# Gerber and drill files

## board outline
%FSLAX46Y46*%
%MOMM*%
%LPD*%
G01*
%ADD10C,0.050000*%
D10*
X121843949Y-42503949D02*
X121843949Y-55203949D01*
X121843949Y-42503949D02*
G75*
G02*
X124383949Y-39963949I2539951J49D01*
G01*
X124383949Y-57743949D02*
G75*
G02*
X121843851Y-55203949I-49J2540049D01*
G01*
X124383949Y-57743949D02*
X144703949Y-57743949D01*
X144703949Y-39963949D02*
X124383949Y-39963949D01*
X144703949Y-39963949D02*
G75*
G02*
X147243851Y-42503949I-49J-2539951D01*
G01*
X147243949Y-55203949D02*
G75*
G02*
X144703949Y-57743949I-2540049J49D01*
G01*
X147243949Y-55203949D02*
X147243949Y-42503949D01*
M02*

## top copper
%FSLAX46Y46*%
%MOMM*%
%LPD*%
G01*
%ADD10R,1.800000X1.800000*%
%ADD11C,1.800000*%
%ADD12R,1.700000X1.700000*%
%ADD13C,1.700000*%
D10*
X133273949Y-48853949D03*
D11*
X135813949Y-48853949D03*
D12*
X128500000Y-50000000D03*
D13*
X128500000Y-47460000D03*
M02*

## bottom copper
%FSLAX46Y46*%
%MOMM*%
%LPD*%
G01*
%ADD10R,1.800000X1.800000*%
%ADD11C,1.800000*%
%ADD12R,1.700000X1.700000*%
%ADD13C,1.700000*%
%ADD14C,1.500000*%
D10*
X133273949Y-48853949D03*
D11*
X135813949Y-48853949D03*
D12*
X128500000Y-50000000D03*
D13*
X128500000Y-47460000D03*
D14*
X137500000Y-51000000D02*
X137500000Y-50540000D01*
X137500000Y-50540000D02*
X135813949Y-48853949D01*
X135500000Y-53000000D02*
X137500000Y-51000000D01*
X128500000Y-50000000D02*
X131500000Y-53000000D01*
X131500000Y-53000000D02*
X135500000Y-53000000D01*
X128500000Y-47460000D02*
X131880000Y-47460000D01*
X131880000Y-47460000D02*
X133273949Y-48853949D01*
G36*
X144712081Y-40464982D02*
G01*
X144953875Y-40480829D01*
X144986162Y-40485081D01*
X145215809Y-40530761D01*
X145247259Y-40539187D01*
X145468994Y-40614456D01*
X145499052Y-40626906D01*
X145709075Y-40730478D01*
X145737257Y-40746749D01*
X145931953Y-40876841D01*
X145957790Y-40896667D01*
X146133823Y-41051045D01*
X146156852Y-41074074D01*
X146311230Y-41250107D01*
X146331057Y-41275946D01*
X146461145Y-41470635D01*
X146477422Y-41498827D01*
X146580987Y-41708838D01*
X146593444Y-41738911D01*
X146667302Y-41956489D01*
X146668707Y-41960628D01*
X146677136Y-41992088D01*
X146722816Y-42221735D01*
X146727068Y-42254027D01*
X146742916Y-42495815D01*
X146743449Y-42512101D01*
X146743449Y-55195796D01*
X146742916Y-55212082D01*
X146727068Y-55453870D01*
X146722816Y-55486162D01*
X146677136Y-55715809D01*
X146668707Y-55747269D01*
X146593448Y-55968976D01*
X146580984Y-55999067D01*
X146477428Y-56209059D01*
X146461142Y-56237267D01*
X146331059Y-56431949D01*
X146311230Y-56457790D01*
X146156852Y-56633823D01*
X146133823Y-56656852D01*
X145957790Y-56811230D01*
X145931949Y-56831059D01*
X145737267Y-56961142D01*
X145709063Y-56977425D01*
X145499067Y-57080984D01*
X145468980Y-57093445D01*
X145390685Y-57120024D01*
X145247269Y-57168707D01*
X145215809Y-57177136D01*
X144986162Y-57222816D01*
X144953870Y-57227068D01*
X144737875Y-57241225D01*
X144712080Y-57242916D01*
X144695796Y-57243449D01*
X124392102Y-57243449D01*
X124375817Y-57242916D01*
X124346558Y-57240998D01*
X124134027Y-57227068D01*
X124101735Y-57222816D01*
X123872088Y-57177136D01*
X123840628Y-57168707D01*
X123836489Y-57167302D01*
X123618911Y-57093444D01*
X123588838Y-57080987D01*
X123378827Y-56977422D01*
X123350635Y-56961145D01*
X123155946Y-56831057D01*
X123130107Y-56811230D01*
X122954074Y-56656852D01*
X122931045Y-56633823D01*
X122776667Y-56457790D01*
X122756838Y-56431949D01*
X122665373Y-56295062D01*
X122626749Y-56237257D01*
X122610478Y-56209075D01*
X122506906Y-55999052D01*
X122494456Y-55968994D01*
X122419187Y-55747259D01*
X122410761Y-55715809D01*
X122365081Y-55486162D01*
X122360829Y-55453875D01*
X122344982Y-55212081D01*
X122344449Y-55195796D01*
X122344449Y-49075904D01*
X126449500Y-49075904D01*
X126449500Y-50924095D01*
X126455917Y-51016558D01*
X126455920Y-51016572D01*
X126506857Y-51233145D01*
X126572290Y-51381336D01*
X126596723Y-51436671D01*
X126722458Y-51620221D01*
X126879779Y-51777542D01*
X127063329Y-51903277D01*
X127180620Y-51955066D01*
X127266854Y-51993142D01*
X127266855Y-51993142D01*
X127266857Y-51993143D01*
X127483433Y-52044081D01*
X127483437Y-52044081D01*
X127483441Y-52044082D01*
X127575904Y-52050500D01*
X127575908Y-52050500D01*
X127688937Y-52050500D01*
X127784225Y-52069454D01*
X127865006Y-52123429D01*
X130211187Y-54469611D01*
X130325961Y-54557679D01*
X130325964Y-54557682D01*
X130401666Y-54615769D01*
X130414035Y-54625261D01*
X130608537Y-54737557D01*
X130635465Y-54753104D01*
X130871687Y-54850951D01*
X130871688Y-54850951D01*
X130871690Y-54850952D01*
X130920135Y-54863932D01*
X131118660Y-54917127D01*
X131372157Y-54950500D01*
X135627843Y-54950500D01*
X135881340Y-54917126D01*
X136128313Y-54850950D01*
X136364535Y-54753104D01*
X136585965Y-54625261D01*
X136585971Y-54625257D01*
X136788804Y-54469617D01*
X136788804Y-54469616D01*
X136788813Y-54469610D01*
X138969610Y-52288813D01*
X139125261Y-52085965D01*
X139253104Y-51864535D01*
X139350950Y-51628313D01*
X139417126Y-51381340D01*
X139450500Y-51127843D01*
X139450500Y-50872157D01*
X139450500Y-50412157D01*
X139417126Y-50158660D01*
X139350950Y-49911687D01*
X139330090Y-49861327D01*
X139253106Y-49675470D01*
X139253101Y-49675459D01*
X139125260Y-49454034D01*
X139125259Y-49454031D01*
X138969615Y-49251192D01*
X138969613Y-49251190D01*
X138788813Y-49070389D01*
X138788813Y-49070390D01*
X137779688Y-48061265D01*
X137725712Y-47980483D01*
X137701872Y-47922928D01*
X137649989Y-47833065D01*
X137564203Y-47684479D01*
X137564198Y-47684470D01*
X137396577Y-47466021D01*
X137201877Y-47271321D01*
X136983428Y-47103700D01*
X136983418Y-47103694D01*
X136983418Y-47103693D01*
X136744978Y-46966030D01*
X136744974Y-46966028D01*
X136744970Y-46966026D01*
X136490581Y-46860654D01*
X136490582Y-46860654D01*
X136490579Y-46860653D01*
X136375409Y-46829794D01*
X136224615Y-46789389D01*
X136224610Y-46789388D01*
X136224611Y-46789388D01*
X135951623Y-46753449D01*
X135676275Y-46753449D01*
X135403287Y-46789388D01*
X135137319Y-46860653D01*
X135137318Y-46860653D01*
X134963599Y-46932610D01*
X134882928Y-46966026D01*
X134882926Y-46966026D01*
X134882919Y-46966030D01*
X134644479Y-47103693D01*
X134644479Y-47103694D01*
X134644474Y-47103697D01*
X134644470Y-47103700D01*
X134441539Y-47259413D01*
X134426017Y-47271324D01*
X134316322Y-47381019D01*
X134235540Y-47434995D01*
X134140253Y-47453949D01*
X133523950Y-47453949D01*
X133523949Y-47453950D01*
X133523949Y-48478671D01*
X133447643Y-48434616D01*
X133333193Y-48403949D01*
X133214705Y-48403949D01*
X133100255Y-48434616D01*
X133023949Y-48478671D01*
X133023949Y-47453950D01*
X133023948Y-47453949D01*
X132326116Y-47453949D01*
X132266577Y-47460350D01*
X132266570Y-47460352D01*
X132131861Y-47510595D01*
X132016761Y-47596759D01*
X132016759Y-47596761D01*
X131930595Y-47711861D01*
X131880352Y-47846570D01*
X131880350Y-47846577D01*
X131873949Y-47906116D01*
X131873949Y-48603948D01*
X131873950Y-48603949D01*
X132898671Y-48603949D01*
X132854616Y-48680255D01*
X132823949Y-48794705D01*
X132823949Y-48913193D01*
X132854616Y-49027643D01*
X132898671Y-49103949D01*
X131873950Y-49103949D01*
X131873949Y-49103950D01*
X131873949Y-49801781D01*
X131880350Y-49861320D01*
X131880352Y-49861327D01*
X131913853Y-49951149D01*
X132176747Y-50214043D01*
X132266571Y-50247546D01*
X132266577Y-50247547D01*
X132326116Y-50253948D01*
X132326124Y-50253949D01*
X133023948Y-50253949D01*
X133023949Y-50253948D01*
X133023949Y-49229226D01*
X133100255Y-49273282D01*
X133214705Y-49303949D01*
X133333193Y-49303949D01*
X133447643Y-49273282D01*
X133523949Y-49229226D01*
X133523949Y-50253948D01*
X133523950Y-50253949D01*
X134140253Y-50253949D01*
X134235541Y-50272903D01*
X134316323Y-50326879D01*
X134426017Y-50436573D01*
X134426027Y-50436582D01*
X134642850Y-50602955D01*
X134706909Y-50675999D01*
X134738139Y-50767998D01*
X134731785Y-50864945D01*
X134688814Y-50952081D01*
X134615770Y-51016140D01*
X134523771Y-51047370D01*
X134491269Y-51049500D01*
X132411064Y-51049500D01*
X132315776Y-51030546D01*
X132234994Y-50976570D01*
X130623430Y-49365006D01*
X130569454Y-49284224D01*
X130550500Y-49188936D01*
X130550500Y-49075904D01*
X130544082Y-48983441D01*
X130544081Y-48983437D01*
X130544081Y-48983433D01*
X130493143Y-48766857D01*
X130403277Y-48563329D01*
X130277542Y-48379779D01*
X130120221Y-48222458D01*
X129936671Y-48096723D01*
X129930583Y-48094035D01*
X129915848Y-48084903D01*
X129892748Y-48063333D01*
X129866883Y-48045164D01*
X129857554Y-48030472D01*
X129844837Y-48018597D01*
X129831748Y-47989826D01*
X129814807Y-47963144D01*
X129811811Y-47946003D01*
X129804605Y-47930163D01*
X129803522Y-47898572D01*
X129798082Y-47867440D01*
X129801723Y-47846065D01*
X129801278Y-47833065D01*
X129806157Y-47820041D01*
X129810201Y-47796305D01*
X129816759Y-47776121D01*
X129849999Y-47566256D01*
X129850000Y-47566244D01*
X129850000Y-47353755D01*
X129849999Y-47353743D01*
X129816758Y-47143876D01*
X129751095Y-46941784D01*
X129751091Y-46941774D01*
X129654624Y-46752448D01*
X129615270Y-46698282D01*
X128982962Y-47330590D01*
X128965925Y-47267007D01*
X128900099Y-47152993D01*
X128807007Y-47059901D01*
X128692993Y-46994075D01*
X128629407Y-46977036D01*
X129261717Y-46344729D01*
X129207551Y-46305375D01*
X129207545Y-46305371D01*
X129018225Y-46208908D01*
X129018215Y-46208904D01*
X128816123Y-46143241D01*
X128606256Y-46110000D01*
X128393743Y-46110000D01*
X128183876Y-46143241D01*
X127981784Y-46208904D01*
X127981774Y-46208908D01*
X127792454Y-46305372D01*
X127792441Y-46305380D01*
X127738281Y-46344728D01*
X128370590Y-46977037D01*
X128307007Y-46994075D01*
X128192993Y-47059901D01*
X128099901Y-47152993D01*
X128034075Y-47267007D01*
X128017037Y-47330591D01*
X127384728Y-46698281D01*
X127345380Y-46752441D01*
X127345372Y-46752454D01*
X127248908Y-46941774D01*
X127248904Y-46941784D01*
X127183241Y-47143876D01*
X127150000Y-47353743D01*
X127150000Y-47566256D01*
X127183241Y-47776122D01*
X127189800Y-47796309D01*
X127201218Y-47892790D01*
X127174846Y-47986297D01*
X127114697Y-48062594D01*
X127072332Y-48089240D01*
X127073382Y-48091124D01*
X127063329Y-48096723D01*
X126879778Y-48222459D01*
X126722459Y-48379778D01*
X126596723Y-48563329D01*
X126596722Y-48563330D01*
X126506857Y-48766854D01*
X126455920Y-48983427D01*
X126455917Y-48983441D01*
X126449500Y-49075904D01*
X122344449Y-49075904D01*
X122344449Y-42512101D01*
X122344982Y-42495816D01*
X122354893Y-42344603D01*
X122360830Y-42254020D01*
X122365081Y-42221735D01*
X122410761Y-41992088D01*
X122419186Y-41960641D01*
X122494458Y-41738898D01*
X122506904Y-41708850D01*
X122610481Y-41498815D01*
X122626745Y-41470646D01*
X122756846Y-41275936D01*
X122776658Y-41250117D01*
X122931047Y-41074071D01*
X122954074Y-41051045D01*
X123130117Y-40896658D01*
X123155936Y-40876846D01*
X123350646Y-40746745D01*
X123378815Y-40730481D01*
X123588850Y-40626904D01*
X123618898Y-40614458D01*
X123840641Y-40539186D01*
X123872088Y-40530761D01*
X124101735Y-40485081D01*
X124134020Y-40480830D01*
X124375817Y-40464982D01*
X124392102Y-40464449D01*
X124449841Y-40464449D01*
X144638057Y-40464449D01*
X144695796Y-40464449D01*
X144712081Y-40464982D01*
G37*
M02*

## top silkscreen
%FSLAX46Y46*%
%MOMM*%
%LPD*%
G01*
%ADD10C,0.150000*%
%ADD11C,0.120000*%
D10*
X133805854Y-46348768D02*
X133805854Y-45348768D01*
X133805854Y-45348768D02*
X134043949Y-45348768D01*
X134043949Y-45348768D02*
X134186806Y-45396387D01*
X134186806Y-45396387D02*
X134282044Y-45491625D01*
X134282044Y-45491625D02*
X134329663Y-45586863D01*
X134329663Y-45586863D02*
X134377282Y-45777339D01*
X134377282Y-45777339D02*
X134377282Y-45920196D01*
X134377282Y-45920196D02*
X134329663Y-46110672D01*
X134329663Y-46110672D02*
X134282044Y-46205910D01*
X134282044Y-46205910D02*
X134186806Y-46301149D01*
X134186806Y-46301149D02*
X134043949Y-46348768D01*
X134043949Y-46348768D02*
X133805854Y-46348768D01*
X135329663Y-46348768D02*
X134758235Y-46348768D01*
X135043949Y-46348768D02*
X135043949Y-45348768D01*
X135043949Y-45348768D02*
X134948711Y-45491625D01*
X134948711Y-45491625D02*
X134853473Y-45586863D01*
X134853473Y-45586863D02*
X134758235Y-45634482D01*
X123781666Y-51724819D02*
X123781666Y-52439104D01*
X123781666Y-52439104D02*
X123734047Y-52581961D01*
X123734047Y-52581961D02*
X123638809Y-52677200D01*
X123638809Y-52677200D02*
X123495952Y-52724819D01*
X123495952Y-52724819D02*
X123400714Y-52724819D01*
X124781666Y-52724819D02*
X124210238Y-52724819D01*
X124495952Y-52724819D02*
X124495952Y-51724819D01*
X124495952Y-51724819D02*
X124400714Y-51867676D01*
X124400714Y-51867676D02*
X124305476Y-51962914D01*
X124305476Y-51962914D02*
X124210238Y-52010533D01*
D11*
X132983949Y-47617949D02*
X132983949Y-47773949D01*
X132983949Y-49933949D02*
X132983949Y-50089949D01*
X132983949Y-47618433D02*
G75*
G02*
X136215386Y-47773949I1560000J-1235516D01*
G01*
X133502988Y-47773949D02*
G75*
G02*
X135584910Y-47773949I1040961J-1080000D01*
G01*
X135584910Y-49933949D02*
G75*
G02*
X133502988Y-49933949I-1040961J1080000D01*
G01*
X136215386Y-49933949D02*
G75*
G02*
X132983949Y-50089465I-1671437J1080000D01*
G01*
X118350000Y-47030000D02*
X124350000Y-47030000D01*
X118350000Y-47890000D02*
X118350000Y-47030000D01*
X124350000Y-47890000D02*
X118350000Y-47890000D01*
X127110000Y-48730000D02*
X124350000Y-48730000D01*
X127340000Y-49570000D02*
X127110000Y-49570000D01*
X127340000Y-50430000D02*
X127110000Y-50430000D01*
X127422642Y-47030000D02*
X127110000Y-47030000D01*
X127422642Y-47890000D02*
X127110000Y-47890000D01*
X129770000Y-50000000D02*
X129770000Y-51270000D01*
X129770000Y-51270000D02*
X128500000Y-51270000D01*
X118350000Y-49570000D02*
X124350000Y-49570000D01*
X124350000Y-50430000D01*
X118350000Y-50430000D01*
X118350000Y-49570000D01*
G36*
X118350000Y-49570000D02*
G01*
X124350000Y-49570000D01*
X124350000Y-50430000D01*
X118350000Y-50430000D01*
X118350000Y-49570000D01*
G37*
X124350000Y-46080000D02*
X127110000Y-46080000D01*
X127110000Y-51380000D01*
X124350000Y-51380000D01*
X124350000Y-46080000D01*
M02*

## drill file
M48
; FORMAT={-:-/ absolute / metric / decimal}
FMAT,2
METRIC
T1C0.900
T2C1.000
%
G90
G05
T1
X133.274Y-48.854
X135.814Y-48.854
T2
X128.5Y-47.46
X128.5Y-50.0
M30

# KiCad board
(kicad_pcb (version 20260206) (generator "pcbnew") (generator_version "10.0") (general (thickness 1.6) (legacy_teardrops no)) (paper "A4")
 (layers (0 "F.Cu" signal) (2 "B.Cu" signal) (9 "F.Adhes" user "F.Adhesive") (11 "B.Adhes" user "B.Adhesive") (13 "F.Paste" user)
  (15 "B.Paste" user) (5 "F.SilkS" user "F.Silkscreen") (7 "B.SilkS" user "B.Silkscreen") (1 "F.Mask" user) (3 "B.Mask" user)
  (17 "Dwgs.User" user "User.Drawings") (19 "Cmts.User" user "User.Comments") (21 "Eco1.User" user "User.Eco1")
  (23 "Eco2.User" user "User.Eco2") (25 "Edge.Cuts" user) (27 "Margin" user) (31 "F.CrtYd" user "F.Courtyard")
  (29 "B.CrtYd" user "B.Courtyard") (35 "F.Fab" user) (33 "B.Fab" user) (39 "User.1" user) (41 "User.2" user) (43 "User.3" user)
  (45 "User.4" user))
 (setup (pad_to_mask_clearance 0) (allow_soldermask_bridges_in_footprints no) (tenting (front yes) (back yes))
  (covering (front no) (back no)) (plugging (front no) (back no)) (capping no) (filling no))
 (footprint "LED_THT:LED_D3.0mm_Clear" (layer "F.Cu") (at 133.273949 48.853949)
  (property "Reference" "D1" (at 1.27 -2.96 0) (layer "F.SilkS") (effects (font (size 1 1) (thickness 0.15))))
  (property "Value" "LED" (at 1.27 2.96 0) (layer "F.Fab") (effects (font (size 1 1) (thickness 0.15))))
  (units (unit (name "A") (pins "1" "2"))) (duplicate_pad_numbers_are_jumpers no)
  (fp_line (start -0.29 -1.236) (end -0.29 -1.08) (stroke (width 0.12) (type solid)) (layer "F.SilkS"))
  (fp_line (start -0.29 1.08) (end -0.29 1.236) (stroke (width 0.12) (type solid)) (layer "F.SilkS"))
  (fp_arc (start -0.29 -1.235516) (mid 1.36566 -1.987699) (end 2.941437 -1.08) (stroke (width 0.12) (type solid)) (layer "F.SilkS"))
  (fp_arc (start 0.229039 -1.08) (mid 1.27 -1.5) (end 2.310961 -1.08) (stroke (width 0.12) (type solid)) (layer "F.SilkS"))
  (fp_arc (start 2.310961 1.08) (mid 1.27 1.5) (end 0.229039 1.08) (stroke (width 0.12) (type solid)) (layer "F.SilkS"))
  (fp_arc (start 2.941437 1.08) (mid 1.36566 1.987699) (end -0.29 1.235516) (stroke (width 0.12) (type solid)) (layer "F.SilkS"))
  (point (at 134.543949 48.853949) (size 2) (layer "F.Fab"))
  (pad "1" thru_hole rect (at 0 0) (size 1.8 1.8) (drill 0.9) (layers "*.Cu" "*.Mask") (remove_unused_layers no) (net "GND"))
  (pad "2" thru_hole circle (at 2.54 0) (size 1.8 1.8) (drill 0.9) (layers "*.Cu" "*.Mask") (remove_unused_layers no) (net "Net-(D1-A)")))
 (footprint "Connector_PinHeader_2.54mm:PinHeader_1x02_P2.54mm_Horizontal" (layer "F.Cu") (at 128.5 50 180)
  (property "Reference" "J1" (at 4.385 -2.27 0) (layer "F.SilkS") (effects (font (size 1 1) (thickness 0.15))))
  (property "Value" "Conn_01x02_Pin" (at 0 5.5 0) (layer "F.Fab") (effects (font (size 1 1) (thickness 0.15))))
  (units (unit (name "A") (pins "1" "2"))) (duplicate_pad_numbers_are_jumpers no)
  (fp_line (start 10.15 2.97) (end 4.15 2.97) (stroke (width 0.12) (type solid)) (layer "F.SilkS"))
  (fp_line (start 10.15 2.11) (end 10.15 2.97) (stroke (width 0.12) (type solid)) (layer "F.SilkS"))
  (fp_line (start 4.15 2.11) (end 10.15 2.11) (stroke (width 0.12) (type solid)) (layer "F.SilkS"))
  (fp_line (start 1.39 1.27) (end 4.15 1.27) (stroke (width 0.12) (type solid)) (layer "F.SilkS"))
  (fp_line (start 1.16 0.43) (end 1.39 0.43) (stroke (width 0.12) (type solid)) (layer "F.SilkS"))
  (fp_line (start 1.16 -0.43) (end 1.39 -0.43) (stroke (width 0.12) (type solid)) (layer "F.SilkS"))
  (fp_line (start 1.077358 2.97) (end 1.39 2.97) (stroke (width 0.12) (type solid)) (layer "F.SilkS"))
  (fp_line (start 1.077358 2.11) (end 1.39 2.11) (stroke (width 0.12) (type solid)) (layer "F.SilkS"))
  (fp_line (start -1.27 0) (end -1.27 -1.27) (stroke (width 0.12) (type solid)) (layer "F.SilkS"))
  (fp_line (start -1.27 -1.27) (end 0 -1.27) (stroke (width 0.12) (type solid)) (layer "F.SilkS"))
  (fp_rect (start 4.15 -0.43) (end 10.15 0.43) (stroke (width 0.12) (type solid)) (fill yes) (layer "F.SilkS"))
  (fp_rect (start 1.39 -1.38) (end 4.15 3.92) (stroke (width 0.12) (type solid)) (fill no) (layer "F.SilkS"))
  (pad "1" thru_hole rect (at 0 0 180) (size 1.7 1.7) (drill 1) (layers "*.Cu" "*.Mask") (remove_unused_layers no) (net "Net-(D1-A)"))
  (pad "2" thru_hole circle (at 0 2.54 180) (size 1.7 1.7) (drill 1) (layers "*.Cu" "*.Mask") (remove_unused_layers no) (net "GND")))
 (gr_line (start 121.843949 42.503949) (end 121.843949 55.203949) (stroke (width 0.05) (type solid)) (layer "Edge.Cuts"))
 (gr_arc (start 121.843949 42.503949) (mid 122.587898 40.707898) (end 124.383949 39.963949) (stroke (width 0.05) (type solid))
  (layer "Edge.Cuts"))
 (gr_arc (start 124.383949 57.743949) (mid 122.587898 57) (end 121.843949 55.203949) (stroke (width 0.05) (type solid)) (layer "Edge.Cuts"))
 (gr_line (start 124.383949 57.743949) (end 144.703949 57.743949) (stroke (width 0.05) (type solid)) (layer "Edge.Cuts"))
 (gr_line (start 144.703949 39.963949) (end 124.383949 39.963949) (stroke (width 0.05) (type solid)) (layer "Edge.Cuts"))
 (gr_arc (start 144.703949 39.963949) (mid 146.5 40.707898) (end 147.243949 42.503949) (stroke (width 0.05) (type solid))
  (layer "Edge.Cuts"))
 (gr_arc (start 147.243949 55.203949) (mid 146.5 57) (end 144.703949 57.743949) (stroke (width 0.05) (type solid)) (layer "Edge.Cuts"))
 (gr_line (start 147.243949 55.203949) (end 147.243949 42.503949) (stroke (width 0.05) (type solid)) (layer "Edge.Cuts"))
 (segment (start 137.5 51) (end 137.5 50.54) (width 1.5) (layer "B.Cu") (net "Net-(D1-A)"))
 (segment (start 137.5 50.54) (end 135.813949 48.853949) (width 1.5) (layer "B.Cu") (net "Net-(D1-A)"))
 (segment (start 135.5 53) (end 137.5 51) (width 1.5) (layer "B.Cu") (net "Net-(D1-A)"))
 (segment (start 128.5 50) (end 131.5 53) (width 1.5) (layer "B.Cu") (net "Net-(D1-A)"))
 (segment (start 131.5 53) (end 135.5 53) (width 1.5) (layer "B.Cu") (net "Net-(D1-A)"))
 (segment (start 128.5 47.46) (end 131.88 47.46) (width 1.5) (layer "B.Cu") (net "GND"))
 (segment (start 131.88 47.46) (end 133.273949 48.853949) (width 1.5) (layer "B.Cu") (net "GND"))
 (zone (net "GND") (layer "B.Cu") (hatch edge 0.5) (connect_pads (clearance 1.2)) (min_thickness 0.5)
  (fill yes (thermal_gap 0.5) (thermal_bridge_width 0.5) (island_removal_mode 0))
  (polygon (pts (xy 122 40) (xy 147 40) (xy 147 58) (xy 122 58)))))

